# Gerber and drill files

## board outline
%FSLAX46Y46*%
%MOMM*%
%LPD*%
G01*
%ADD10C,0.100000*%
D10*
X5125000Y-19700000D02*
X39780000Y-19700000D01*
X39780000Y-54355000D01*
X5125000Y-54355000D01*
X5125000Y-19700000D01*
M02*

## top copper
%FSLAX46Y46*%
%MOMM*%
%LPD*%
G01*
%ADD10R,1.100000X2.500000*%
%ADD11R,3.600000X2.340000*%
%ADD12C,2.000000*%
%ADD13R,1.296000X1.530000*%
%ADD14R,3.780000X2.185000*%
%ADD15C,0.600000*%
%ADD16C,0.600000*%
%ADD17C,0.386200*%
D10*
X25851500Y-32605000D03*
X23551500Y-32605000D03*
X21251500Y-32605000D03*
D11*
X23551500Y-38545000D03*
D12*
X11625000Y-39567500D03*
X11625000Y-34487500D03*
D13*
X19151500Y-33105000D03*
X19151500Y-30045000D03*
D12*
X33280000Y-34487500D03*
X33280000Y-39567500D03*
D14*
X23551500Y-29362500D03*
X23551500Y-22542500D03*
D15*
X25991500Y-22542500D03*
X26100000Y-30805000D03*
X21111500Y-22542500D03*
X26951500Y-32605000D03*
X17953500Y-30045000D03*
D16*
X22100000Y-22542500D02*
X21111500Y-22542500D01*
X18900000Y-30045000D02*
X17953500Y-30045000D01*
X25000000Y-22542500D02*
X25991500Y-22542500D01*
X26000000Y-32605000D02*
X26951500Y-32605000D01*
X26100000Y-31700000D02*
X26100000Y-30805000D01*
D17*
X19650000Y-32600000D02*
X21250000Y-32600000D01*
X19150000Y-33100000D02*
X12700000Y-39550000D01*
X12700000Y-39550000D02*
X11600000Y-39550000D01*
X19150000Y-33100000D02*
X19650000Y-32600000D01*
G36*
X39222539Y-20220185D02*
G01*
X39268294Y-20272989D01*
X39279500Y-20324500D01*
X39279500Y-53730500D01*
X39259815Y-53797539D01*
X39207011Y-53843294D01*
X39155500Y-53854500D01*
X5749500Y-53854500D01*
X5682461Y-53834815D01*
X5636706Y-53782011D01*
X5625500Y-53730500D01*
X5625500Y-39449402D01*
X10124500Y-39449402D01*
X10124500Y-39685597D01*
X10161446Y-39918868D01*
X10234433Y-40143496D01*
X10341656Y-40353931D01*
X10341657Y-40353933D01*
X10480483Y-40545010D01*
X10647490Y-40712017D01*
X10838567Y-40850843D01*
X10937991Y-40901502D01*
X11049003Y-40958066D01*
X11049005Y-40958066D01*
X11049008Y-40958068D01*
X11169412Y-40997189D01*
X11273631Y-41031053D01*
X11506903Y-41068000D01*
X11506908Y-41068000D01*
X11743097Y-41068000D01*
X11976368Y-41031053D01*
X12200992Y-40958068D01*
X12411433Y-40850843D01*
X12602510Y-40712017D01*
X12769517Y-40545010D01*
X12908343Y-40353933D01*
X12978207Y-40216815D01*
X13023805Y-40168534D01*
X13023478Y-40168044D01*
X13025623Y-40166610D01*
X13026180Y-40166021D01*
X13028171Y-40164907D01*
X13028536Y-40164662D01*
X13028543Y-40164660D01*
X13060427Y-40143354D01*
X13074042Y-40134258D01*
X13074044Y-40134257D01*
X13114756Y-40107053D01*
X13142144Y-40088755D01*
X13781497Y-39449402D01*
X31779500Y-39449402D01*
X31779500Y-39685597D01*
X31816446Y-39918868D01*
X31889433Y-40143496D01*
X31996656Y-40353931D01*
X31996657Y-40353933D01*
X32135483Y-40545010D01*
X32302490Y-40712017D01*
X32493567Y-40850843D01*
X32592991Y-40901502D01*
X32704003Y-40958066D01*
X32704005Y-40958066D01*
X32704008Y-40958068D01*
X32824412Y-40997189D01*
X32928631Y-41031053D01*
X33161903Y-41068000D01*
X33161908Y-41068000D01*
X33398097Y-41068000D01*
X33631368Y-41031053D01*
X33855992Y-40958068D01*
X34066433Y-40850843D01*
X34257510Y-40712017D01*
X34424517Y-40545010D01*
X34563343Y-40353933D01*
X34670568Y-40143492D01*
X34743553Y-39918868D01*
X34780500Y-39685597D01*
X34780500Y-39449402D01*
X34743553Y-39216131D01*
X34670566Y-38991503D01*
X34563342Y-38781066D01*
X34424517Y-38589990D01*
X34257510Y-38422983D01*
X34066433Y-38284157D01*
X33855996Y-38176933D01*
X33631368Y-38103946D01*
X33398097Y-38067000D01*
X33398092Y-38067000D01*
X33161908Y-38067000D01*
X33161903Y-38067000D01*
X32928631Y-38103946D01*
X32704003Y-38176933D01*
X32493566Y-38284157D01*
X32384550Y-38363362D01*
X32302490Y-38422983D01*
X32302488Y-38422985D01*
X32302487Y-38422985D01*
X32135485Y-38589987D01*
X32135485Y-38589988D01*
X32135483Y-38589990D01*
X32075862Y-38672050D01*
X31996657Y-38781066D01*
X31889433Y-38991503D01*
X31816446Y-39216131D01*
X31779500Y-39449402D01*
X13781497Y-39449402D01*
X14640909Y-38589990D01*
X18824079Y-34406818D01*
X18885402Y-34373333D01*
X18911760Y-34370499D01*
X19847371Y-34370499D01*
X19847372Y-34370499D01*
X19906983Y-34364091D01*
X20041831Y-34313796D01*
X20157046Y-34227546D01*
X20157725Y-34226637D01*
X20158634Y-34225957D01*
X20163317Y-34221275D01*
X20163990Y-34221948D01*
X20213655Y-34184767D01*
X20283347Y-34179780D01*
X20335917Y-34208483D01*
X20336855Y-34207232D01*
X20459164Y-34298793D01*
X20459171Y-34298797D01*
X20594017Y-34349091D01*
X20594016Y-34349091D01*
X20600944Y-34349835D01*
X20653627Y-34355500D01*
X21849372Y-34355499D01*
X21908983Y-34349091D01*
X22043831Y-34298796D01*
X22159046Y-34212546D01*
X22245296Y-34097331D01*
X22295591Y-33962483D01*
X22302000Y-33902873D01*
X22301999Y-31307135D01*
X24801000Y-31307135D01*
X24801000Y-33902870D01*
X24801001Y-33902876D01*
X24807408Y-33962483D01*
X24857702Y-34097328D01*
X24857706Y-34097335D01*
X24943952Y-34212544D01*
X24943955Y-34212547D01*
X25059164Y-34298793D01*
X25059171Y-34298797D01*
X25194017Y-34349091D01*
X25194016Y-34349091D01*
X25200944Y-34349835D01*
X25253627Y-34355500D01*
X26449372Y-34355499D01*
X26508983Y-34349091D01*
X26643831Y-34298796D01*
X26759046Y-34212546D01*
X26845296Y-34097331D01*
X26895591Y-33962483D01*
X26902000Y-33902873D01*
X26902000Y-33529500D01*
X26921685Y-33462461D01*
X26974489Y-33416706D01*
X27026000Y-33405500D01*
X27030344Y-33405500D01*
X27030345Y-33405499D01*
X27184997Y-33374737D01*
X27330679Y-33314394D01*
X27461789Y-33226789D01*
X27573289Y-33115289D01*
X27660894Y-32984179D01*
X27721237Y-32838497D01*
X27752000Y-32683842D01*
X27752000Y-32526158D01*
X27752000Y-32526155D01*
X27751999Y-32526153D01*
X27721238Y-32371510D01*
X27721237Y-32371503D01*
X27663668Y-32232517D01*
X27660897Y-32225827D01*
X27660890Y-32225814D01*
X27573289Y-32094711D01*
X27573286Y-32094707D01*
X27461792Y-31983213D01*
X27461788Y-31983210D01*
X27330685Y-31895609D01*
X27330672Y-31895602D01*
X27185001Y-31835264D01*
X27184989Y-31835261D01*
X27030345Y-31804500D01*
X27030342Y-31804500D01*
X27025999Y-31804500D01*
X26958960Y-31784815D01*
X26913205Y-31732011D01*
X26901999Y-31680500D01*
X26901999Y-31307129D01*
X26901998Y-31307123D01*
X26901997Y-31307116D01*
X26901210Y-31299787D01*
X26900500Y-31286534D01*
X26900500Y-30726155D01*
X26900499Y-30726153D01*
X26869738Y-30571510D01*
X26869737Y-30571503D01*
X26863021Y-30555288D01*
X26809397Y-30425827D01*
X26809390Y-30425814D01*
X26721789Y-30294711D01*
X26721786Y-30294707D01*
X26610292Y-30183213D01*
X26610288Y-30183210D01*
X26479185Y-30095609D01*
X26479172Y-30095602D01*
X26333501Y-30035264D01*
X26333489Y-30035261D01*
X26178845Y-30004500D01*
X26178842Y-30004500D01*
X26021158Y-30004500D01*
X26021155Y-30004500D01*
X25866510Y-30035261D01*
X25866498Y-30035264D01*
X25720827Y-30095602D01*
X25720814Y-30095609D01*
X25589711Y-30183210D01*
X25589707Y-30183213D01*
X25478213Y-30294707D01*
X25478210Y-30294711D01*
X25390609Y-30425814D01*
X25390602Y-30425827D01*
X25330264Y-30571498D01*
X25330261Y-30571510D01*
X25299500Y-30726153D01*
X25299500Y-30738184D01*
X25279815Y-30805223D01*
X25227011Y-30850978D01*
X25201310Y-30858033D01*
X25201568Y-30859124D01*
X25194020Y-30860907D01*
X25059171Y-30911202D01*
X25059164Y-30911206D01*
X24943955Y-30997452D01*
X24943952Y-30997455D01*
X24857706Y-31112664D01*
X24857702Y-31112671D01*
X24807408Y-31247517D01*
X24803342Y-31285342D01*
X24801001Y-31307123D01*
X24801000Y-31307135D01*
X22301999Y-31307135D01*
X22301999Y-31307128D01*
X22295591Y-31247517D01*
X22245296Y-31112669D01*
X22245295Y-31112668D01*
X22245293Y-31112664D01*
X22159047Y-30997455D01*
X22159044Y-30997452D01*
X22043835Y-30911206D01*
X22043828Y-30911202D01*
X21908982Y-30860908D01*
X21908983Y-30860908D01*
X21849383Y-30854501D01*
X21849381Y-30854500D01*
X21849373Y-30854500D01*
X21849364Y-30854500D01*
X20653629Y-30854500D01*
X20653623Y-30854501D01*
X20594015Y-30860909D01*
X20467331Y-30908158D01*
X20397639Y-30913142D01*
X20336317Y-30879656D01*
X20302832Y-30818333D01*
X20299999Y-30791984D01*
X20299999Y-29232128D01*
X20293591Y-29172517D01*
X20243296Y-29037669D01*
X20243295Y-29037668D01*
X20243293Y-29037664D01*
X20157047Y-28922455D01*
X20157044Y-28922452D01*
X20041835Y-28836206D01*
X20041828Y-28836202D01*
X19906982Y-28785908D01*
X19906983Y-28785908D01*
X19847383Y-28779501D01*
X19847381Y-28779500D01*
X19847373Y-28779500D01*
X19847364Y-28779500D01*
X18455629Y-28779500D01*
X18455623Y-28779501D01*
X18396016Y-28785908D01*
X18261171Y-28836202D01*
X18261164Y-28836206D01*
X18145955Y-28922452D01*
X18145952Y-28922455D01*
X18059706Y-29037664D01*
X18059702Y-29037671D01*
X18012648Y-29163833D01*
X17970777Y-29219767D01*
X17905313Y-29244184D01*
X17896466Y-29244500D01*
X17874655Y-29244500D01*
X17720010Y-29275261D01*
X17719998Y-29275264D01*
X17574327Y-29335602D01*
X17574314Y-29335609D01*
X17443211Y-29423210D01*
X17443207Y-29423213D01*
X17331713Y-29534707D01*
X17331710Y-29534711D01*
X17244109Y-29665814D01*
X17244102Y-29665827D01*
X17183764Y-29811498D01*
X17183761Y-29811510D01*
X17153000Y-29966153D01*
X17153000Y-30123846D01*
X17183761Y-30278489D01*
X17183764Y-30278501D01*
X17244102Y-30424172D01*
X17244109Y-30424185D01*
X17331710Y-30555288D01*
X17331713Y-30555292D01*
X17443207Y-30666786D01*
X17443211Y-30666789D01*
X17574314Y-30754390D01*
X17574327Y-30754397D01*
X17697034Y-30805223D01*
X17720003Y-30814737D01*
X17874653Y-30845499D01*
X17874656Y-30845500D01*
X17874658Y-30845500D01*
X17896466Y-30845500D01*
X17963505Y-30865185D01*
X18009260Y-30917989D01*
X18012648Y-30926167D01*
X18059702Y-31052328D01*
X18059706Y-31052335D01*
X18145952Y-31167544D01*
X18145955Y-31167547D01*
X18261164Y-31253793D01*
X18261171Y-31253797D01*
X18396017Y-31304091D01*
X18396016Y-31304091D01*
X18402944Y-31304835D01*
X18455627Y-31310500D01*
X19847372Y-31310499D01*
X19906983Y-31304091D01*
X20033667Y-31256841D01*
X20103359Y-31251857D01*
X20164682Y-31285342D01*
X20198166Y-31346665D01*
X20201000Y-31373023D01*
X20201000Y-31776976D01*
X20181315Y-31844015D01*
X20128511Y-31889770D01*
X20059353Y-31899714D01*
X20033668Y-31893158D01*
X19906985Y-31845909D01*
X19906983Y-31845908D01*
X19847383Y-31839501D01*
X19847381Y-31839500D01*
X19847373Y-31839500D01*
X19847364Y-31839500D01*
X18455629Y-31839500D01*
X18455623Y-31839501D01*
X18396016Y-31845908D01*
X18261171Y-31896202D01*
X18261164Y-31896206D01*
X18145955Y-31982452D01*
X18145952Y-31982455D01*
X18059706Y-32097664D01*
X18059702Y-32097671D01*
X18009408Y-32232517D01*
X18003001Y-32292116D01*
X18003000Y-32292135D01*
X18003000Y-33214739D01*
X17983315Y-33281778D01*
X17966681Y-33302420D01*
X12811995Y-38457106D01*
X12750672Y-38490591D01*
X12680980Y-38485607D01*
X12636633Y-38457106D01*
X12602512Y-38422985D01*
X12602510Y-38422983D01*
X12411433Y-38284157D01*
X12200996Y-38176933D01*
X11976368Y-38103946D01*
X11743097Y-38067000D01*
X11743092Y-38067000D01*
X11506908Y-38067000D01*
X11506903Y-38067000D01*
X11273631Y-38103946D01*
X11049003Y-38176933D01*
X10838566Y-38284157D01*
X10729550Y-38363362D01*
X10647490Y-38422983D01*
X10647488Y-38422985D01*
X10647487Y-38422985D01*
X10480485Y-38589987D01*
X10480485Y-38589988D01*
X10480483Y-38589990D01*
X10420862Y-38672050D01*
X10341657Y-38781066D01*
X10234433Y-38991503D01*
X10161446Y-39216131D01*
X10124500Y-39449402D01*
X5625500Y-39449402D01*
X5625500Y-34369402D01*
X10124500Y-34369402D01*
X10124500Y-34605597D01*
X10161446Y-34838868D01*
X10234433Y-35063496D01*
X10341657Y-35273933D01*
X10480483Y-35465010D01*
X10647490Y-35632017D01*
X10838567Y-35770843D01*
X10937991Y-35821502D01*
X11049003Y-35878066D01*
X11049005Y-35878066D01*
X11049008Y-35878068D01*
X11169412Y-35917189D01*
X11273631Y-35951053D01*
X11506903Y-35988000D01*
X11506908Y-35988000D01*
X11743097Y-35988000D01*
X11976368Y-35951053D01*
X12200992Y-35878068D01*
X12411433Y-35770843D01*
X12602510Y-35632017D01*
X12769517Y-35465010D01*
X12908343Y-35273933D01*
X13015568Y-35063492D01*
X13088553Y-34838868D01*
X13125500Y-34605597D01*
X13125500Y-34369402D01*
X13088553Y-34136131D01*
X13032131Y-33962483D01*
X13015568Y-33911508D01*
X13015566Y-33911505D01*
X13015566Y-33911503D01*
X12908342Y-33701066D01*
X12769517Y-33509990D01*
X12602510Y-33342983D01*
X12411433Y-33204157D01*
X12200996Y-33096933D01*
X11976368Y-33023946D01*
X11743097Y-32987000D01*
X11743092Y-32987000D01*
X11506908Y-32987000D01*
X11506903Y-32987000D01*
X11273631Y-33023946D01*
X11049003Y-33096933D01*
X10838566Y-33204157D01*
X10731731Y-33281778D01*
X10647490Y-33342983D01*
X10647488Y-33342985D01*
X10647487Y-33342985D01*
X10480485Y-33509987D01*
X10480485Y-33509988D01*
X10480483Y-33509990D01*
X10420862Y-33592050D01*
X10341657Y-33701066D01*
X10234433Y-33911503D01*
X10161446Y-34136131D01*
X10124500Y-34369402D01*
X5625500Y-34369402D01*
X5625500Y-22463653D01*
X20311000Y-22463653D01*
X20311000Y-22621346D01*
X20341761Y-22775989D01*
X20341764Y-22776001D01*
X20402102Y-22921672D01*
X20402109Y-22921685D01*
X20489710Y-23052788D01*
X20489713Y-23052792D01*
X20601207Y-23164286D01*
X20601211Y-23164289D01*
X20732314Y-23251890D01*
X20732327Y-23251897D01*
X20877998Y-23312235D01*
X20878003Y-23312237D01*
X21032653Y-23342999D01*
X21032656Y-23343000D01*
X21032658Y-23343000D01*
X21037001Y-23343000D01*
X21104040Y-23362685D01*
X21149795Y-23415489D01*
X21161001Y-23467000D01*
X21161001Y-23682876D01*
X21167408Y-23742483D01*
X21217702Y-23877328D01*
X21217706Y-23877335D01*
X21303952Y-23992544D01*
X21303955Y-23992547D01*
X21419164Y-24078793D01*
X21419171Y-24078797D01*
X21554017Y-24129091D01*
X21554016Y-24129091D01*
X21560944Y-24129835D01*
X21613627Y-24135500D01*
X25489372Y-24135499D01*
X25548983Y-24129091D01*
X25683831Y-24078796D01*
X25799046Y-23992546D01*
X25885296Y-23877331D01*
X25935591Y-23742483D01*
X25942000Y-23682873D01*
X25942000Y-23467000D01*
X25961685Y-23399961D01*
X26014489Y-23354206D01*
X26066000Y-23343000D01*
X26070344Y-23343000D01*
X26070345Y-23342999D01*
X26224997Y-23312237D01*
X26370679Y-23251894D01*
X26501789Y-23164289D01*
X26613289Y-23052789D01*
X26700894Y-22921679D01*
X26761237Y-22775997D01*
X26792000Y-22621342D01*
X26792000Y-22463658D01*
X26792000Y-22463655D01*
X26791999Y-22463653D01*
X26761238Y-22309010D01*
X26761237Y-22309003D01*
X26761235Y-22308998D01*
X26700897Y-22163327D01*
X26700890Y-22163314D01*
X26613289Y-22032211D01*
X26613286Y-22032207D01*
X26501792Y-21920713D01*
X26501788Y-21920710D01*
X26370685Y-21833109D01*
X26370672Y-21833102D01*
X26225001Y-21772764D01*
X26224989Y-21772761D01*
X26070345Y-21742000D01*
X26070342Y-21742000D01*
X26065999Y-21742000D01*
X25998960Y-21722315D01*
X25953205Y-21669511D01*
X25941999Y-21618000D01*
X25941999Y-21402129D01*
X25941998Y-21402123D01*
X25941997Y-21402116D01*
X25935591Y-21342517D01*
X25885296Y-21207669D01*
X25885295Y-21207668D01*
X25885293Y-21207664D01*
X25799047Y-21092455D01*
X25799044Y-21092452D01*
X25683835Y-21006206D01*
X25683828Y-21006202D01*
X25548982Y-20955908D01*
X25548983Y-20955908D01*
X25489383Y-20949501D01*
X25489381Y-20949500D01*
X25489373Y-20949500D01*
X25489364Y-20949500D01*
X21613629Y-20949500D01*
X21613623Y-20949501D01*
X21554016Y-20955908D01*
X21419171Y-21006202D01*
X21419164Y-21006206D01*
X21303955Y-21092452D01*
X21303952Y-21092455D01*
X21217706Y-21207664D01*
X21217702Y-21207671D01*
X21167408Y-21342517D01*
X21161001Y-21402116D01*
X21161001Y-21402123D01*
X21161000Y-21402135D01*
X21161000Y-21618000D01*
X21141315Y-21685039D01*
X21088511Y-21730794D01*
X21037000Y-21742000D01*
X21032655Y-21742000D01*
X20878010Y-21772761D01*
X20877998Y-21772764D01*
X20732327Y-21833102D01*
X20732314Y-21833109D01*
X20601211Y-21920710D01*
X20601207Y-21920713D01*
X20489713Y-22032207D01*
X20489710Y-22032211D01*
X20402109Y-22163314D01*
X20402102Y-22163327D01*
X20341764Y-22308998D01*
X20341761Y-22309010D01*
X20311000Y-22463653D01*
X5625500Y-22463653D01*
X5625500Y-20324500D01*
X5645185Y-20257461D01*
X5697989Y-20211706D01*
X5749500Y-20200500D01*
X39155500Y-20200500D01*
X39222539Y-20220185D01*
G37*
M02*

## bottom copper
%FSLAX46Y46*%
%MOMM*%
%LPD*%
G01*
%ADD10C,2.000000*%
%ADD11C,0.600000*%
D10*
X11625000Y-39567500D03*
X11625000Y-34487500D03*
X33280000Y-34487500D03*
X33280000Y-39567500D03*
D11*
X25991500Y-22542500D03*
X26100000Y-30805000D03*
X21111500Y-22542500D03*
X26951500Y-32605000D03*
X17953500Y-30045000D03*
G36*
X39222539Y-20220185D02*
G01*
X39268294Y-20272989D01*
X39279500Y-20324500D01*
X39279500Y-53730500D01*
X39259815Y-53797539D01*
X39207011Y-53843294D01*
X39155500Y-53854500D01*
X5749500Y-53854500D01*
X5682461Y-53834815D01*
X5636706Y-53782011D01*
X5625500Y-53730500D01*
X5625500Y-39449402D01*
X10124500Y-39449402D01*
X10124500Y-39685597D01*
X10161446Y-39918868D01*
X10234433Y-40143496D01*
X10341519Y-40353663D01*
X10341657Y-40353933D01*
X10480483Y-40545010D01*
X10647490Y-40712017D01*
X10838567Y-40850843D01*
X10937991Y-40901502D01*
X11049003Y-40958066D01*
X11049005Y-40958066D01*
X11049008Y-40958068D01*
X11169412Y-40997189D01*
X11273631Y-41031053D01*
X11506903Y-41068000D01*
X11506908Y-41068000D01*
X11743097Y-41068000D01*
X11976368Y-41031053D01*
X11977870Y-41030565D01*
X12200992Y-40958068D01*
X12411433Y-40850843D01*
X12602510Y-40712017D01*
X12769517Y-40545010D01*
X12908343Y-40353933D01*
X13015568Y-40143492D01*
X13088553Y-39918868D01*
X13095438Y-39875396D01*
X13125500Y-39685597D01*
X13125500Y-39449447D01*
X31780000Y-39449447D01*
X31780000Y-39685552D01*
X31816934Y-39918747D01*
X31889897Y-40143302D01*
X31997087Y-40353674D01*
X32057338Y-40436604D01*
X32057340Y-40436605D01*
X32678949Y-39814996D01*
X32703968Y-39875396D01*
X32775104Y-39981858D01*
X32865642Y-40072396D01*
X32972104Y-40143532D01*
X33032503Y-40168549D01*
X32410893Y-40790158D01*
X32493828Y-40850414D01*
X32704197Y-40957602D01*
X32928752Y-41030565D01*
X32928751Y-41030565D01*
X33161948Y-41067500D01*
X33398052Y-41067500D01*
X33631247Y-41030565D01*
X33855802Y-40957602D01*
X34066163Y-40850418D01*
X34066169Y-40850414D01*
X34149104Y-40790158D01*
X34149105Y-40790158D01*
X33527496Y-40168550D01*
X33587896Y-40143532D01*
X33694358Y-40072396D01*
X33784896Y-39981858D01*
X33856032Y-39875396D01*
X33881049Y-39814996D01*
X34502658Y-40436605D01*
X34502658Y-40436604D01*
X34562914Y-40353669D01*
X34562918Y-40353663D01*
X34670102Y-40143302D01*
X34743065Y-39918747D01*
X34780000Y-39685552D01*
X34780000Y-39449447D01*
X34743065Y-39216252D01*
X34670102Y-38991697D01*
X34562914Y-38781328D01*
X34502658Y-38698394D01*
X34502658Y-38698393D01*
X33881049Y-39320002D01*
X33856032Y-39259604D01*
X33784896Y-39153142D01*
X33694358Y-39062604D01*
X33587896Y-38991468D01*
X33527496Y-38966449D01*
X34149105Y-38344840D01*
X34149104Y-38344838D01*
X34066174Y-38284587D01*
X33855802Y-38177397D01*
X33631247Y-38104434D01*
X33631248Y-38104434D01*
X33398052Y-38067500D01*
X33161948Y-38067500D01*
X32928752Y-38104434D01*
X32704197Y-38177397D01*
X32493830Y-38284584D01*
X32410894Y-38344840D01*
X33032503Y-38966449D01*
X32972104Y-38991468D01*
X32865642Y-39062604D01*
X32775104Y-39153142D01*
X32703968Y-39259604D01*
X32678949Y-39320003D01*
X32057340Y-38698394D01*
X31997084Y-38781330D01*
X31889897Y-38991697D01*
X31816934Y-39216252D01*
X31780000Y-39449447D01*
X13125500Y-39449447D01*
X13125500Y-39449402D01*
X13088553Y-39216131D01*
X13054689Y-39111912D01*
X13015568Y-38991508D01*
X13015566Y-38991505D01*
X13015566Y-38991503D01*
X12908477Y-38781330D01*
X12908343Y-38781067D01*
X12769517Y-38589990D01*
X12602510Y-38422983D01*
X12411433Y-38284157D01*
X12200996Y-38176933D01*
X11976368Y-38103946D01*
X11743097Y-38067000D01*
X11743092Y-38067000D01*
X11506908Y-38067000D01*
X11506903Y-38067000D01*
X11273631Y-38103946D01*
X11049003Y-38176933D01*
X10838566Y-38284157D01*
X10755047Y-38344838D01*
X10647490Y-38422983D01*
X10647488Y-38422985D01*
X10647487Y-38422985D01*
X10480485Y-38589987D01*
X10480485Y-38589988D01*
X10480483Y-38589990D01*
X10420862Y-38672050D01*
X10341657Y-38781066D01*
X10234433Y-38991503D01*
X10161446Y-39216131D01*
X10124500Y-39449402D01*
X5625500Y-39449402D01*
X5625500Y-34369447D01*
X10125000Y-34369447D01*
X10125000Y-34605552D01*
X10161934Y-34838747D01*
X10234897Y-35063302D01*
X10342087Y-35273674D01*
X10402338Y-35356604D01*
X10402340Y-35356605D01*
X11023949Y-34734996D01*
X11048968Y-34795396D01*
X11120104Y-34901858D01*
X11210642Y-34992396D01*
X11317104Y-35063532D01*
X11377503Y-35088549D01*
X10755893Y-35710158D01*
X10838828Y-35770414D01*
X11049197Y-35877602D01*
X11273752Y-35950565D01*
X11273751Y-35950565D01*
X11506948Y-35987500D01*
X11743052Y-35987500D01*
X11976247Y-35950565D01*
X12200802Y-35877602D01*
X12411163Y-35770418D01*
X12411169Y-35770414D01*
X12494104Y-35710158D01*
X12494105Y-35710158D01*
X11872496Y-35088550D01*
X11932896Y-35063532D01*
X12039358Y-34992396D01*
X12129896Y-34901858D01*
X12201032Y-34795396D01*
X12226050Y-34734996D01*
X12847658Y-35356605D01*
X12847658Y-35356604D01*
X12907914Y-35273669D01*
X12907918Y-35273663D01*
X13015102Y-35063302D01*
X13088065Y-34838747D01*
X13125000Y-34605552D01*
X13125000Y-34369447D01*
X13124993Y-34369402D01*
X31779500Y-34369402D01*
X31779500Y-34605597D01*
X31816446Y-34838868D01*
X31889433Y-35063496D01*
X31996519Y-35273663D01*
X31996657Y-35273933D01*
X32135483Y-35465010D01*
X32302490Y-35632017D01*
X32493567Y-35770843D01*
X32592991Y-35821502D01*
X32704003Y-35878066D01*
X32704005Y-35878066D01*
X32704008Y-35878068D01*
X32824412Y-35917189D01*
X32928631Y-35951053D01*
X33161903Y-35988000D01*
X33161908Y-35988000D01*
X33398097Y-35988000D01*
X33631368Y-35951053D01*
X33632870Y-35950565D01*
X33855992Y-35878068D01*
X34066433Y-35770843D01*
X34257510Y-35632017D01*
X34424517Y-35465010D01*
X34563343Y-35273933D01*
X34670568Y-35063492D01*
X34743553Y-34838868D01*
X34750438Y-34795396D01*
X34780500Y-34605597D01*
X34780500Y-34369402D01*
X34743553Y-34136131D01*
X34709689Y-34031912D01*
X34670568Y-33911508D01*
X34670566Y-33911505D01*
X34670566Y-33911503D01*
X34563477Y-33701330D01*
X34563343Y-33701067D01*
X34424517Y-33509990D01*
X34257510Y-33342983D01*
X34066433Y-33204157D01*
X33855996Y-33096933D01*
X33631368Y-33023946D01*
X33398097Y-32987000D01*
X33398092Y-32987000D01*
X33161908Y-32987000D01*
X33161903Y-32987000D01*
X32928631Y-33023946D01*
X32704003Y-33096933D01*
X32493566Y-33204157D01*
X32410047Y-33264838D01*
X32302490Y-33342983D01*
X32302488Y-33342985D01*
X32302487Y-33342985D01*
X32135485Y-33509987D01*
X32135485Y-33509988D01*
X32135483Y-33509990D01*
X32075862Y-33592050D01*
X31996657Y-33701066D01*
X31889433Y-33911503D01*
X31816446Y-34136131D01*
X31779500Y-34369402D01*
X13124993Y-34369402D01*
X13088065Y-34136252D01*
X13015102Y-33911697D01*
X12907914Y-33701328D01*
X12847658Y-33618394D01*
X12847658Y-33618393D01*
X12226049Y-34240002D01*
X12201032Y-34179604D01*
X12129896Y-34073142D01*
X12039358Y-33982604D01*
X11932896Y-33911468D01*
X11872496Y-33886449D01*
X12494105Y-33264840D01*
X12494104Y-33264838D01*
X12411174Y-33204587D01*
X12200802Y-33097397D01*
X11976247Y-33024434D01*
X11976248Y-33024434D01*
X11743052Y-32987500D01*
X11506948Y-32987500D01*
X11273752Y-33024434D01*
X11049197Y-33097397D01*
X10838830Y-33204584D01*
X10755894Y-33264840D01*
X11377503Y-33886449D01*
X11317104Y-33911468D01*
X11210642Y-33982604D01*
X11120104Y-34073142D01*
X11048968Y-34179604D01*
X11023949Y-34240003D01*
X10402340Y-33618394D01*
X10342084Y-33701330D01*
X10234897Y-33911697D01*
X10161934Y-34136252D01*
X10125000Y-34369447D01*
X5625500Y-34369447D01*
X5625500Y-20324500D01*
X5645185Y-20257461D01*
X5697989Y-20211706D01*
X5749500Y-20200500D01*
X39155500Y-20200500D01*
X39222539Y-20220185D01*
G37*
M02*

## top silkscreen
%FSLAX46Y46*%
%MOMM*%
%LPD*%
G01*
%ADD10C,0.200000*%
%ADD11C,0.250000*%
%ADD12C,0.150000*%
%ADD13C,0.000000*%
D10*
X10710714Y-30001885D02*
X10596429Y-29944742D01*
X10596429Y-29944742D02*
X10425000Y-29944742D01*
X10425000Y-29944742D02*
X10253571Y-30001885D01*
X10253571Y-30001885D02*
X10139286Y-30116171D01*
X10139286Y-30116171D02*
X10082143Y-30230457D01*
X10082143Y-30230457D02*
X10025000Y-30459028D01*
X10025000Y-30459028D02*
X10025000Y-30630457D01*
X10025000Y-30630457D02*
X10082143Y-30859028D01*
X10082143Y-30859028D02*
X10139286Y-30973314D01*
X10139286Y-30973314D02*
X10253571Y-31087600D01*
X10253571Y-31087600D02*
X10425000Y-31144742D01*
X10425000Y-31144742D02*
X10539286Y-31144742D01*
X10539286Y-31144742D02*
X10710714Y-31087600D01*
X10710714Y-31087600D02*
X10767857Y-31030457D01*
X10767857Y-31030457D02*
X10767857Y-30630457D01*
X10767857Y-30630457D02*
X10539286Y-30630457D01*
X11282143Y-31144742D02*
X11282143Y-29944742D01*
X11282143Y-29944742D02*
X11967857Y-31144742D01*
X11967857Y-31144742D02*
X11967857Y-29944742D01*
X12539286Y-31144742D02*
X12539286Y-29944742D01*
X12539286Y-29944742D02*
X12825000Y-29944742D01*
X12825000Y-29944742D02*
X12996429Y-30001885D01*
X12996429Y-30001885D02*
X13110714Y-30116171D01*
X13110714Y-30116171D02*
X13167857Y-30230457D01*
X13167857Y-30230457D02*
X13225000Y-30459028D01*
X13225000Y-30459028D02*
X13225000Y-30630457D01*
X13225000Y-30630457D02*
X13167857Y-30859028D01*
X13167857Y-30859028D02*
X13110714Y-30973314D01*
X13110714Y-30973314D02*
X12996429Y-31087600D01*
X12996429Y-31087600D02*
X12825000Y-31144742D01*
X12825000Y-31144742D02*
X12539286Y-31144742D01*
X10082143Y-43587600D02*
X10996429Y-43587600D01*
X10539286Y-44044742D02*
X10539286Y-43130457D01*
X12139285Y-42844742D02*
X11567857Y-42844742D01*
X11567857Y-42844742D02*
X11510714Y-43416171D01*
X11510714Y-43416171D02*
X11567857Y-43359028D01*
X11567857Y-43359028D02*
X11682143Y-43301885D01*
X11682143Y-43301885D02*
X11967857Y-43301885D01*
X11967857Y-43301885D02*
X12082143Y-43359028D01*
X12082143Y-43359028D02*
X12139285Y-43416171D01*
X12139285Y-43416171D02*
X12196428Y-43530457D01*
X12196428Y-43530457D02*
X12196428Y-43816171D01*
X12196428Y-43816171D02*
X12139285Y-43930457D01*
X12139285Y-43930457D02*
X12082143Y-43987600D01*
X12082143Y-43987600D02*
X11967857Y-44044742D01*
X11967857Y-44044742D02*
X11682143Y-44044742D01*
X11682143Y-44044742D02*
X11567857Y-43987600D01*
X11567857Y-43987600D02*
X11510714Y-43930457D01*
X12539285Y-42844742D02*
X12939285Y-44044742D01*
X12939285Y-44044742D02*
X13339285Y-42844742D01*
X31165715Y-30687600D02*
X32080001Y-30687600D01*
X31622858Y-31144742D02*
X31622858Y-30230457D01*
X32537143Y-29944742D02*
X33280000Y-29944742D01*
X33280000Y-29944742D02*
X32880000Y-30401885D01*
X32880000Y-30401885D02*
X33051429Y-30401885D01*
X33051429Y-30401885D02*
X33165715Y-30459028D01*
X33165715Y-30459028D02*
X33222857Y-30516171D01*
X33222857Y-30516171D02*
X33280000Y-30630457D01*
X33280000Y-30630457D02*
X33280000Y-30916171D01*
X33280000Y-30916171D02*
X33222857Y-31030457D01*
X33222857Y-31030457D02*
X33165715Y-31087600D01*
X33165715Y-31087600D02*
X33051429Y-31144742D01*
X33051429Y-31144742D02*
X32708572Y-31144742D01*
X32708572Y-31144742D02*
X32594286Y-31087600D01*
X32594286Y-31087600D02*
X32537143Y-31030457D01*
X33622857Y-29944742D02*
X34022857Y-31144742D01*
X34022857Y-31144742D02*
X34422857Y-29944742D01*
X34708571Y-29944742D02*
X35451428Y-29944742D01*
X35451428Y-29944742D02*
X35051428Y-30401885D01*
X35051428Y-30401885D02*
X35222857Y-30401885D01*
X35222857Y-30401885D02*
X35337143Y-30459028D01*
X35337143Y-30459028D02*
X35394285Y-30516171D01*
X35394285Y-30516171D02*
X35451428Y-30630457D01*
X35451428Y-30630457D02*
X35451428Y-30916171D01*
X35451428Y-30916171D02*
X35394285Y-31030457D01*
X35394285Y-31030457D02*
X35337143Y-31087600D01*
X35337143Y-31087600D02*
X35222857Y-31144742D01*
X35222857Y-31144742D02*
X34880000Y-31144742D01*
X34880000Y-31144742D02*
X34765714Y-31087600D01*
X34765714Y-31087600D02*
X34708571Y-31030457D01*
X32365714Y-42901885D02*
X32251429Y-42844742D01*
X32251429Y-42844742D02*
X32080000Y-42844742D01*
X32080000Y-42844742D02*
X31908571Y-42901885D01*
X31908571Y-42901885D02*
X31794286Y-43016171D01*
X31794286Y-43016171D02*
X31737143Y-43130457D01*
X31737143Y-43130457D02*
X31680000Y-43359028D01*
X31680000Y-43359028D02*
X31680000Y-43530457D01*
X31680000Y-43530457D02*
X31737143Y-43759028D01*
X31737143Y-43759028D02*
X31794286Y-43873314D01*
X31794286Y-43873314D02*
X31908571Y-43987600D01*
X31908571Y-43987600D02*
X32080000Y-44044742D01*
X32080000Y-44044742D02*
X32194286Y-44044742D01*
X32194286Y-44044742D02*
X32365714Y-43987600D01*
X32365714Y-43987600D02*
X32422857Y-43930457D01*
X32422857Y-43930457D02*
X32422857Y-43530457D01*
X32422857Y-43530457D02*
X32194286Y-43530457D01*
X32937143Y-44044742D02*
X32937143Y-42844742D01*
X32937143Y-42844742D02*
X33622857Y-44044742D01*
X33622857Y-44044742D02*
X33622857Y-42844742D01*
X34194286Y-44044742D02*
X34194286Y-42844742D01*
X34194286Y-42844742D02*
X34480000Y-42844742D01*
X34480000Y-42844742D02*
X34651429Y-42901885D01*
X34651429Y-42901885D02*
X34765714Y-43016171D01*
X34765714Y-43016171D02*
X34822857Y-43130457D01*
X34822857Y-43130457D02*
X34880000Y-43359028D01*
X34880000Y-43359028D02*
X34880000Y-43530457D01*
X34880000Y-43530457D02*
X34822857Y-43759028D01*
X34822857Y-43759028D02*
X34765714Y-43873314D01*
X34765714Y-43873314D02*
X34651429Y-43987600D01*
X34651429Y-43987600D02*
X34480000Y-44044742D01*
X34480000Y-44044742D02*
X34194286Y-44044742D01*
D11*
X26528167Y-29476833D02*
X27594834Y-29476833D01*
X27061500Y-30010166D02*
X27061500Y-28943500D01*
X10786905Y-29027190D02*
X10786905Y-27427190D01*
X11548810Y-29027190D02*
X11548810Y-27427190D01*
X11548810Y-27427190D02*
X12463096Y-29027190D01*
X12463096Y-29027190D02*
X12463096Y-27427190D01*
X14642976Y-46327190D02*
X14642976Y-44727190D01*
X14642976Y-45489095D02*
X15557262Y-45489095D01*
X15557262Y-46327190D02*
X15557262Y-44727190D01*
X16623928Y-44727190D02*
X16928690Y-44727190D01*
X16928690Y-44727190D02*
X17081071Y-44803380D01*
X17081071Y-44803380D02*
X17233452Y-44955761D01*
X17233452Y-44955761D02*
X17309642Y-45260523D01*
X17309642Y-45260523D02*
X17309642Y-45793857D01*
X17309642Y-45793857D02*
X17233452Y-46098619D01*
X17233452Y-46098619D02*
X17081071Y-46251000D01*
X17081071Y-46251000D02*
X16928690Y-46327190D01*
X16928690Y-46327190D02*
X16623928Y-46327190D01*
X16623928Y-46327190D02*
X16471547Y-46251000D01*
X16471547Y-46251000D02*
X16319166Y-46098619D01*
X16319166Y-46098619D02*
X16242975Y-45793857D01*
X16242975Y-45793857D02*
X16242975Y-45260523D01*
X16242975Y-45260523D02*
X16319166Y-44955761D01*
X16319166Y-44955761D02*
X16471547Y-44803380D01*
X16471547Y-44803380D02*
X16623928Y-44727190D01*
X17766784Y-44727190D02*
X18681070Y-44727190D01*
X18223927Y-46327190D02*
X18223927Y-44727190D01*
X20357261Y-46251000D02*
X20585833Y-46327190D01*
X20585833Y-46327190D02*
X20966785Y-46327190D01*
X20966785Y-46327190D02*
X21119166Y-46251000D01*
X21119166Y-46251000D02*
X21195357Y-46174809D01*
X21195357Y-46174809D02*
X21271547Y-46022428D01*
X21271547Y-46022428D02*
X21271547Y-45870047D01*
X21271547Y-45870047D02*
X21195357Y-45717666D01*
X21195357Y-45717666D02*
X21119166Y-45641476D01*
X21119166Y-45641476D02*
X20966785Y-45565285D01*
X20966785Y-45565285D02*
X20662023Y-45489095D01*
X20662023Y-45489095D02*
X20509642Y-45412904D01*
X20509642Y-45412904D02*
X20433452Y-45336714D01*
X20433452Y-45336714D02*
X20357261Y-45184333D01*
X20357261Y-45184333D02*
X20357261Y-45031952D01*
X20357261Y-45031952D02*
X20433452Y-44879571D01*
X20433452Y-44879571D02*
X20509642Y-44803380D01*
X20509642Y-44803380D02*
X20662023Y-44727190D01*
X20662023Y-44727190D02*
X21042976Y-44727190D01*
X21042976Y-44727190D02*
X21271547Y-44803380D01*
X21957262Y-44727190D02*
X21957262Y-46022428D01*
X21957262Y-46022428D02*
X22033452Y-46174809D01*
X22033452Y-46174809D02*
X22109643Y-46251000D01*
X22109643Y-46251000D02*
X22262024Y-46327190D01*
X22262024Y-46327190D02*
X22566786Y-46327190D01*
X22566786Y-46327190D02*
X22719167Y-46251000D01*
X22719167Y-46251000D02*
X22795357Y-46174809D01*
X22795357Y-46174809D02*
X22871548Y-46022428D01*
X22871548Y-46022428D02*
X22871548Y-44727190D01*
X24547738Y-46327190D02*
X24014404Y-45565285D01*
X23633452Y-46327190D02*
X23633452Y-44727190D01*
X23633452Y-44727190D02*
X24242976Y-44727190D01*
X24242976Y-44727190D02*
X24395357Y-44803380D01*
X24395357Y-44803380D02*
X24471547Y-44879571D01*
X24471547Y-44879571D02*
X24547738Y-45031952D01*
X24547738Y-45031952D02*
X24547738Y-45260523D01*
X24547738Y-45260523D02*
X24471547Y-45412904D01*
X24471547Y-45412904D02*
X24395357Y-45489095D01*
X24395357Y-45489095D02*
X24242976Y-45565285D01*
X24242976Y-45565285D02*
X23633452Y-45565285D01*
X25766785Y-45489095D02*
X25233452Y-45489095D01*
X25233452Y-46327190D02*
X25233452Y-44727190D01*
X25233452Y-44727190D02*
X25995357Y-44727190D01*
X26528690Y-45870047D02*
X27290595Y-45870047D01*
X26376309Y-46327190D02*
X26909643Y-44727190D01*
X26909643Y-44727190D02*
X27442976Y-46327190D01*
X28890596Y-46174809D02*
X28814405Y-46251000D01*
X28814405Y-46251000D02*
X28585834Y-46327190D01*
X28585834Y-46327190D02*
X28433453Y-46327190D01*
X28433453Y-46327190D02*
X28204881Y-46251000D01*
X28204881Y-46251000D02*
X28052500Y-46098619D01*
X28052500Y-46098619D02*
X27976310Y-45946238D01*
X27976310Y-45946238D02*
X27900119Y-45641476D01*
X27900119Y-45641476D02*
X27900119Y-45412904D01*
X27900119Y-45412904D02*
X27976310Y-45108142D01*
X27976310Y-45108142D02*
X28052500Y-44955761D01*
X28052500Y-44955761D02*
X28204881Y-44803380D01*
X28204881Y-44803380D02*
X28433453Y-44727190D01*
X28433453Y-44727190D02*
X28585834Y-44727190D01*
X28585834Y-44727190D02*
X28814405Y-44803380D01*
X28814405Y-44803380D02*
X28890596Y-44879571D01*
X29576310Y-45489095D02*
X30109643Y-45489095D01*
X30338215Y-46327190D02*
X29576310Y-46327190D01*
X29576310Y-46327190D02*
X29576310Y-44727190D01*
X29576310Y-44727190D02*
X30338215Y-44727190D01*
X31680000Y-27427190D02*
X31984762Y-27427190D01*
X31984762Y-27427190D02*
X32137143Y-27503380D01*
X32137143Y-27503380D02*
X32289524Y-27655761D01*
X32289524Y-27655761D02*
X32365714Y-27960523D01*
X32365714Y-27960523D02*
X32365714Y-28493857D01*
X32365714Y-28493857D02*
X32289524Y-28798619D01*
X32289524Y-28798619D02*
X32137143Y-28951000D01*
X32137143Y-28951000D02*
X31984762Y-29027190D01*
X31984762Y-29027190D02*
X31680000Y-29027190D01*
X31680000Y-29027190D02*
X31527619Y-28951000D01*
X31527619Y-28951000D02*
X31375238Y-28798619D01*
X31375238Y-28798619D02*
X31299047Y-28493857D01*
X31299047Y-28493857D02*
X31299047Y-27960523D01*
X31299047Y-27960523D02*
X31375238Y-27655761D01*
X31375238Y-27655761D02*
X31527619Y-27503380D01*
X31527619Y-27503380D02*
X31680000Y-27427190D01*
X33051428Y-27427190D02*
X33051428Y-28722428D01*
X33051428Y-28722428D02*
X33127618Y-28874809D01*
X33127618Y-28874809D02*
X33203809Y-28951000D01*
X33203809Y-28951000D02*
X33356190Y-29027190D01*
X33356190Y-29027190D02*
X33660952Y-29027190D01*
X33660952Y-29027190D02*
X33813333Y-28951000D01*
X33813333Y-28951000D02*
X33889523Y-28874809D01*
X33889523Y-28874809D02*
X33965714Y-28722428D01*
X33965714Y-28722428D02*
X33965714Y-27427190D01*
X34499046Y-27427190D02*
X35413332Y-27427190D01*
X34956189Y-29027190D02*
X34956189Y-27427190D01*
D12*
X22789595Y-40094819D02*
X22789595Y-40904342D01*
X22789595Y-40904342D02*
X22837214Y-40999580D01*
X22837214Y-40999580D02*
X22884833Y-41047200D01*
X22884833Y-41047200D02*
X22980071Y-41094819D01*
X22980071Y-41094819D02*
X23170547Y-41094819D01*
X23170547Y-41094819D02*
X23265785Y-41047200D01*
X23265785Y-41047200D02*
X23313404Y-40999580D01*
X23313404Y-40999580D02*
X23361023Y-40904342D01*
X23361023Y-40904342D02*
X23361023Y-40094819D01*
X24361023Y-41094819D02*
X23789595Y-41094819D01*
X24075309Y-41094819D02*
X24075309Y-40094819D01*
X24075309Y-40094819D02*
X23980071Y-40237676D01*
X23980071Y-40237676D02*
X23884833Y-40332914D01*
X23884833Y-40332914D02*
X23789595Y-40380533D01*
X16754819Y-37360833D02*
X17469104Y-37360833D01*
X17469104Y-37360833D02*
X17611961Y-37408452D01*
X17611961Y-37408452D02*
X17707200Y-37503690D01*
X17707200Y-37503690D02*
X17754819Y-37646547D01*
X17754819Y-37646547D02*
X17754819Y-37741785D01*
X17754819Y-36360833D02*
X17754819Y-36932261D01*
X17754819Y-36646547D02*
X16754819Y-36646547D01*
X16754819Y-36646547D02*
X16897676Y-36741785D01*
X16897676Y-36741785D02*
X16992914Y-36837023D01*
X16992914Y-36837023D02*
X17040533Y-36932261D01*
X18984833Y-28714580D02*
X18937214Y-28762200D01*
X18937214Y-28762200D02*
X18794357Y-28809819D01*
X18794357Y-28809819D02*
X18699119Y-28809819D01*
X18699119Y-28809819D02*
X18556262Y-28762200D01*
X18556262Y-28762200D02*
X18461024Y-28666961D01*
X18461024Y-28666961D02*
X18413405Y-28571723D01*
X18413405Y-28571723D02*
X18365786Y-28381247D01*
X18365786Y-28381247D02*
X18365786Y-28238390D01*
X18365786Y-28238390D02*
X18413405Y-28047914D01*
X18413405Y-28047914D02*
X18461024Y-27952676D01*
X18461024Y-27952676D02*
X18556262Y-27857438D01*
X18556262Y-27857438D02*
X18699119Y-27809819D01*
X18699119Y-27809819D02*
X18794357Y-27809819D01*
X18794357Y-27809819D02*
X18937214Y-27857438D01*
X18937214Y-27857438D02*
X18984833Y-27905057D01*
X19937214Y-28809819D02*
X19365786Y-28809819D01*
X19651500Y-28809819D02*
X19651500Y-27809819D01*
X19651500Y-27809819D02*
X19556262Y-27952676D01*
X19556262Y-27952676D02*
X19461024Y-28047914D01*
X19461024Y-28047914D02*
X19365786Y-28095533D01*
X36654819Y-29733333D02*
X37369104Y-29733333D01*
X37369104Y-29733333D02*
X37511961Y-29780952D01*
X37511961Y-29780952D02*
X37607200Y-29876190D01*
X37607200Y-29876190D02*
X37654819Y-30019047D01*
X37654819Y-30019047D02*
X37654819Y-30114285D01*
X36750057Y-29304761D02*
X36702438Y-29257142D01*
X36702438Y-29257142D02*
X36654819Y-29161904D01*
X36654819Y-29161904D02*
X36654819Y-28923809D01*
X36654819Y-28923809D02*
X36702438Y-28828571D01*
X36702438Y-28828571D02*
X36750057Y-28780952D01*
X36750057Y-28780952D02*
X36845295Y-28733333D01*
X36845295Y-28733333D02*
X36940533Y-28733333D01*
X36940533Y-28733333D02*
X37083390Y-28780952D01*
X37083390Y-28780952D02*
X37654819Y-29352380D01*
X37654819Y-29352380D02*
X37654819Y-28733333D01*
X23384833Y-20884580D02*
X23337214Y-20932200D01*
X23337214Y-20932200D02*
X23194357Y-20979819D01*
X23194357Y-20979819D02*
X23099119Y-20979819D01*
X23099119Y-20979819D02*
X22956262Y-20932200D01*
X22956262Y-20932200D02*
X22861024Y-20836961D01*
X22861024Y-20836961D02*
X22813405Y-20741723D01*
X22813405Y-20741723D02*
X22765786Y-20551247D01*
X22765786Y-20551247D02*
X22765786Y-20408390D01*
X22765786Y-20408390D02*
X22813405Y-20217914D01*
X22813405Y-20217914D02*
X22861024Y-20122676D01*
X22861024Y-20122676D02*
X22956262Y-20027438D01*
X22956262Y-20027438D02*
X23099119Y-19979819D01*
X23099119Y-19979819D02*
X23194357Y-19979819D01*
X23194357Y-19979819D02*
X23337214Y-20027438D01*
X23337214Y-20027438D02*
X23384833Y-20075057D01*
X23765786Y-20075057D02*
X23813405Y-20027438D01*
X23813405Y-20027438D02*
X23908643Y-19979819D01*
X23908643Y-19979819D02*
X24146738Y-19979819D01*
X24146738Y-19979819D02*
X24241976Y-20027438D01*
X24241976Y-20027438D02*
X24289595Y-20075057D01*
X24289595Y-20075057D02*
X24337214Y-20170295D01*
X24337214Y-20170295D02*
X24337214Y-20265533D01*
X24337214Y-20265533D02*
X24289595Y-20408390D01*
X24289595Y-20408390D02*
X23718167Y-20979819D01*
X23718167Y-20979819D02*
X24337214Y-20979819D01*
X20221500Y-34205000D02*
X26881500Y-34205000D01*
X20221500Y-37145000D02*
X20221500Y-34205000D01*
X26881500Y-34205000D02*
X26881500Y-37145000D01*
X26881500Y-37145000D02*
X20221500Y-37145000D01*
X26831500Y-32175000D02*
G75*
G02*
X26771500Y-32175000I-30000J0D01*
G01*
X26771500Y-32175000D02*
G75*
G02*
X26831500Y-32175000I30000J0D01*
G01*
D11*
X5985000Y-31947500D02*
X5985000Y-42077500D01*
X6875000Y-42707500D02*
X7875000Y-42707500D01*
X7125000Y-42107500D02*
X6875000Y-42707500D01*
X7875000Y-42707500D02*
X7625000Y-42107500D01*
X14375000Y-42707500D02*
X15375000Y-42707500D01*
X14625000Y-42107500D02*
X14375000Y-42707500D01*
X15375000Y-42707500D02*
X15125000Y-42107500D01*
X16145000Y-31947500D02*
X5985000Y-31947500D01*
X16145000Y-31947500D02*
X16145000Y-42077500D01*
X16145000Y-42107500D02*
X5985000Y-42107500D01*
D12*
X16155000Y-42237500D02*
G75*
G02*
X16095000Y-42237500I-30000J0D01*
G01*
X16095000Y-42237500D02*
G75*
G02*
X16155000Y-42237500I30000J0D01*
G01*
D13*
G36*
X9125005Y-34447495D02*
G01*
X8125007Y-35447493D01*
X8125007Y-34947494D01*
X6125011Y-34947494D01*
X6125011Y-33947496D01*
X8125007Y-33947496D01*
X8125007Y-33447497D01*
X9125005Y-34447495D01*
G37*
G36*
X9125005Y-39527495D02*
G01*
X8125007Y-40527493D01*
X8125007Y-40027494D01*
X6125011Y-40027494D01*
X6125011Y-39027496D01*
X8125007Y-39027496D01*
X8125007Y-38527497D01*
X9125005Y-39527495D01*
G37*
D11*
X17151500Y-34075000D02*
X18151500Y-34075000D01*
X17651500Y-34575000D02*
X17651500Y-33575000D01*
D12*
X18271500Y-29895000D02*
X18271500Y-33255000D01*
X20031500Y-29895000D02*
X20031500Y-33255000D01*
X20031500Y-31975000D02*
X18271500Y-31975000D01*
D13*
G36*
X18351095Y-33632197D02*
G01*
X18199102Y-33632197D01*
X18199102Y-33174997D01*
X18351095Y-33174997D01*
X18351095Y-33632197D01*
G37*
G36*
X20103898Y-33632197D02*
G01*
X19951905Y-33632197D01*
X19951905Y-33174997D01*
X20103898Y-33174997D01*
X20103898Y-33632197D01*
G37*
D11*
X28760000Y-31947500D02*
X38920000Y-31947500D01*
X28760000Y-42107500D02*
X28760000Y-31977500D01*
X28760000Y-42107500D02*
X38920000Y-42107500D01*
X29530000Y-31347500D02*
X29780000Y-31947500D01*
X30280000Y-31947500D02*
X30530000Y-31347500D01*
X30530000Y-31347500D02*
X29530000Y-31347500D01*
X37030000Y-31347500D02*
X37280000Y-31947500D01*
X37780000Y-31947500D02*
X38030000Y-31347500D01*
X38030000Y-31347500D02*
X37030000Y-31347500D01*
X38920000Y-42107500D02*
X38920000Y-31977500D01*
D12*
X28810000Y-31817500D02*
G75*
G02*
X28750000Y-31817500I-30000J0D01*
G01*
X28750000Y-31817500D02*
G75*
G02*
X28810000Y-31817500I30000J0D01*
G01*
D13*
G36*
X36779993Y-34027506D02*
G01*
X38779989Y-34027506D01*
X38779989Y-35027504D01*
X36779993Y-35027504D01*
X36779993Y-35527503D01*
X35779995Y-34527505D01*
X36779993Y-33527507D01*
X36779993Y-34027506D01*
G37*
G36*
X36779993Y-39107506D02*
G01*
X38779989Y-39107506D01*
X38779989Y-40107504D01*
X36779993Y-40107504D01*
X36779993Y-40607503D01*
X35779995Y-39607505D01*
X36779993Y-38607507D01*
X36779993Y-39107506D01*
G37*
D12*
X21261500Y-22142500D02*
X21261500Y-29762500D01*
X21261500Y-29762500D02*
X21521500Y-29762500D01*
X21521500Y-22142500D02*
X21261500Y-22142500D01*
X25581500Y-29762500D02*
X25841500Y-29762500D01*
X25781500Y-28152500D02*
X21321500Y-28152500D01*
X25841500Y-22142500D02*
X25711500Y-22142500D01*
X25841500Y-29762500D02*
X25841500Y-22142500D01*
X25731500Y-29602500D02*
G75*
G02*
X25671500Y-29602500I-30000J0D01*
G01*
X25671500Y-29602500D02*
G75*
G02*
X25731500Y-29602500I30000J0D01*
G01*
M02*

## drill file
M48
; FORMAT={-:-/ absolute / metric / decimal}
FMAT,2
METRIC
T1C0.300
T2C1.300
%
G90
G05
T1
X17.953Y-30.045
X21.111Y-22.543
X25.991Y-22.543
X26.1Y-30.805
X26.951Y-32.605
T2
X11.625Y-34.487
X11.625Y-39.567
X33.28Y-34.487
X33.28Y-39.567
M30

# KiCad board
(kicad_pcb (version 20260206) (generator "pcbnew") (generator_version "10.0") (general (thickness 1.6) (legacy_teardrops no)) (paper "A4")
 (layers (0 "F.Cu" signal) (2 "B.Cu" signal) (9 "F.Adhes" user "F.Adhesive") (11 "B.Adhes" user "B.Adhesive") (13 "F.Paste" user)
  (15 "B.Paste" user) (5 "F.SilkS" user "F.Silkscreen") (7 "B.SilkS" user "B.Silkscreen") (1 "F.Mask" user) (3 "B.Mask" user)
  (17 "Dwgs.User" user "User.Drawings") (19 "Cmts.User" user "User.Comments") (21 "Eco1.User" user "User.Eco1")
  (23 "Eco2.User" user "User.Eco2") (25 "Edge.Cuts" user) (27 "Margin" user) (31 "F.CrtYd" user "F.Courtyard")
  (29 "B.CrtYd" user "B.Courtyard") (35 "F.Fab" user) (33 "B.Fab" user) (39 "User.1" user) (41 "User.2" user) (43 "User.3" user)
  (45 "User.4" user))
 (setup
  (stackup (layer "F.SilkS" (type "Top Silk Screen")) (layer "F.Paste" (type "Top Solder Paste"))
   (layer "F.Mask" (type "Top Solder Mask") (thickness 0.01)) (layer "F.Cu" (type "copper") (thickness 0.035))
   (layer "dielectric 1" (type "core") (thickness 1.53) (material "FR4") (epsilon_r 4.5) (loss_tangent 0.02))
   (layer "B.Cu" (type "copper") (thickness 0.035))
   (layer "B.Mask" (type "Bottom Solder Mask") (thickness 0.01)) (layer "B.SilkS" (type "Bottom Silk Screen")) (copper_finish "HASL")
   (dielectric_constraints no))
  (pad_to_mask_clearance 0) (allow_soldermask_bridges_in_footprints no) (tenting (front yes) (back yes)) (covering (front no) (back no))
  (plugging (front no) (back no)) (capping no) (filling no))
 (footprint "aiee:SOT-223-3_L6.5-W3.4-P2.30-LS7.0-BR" (layer "F.Cu") (at 23.5515 35.575 90)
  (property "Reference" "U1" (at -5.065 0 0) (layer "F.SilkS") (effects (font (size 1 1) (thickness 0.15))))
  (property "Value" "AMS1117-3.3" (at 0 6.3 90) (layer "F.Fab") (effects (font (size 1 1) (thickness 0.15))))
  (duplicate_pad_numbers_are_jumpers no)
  (fp_line (start 1.37 -3.33) (end 1.37 3.33) (stroke (width 0.15) (type solid)) (layer "F.SilkS"))
  (fp_line (start -1.57 -3.33) (end 1.37 -3.33) (stroke (width 0.15) (type solid)) (layer "F.SilkS"))
  (fp_line (start 1.37 3.33) (end -1.57 3.33) (stroke (width 0.15) (type solid)) (layer "F.SilkS"))
  (fp_line (start -1.57 3.33) (end -1.57 -3.33) (stroke (width 0.15) (type solid)) (layer "F.SilkS"))
  (fp_circle (center 3.4 3.25) (end 3.43 3.25) (stroke (width 0.15) (type solid)) (fill no) (layer "F.SilkS"))
  (pad "1" smd rect (at 2.97 2.3 90) (size 2.5 1.1) (layers "F.Cu" "F.Mask" "F.Paste") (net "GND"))
  (pad "2" smd rect (at 2.97 0 90) (size 2.5 1.1) (layers "F.Cu" "F.Mask" "F.Paste") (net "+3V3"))
  (pad "3" smd rect (at 2.97 -2.3 90) (size 2.5 1.1) (layers "F.Cu" "F.Mask" "F.Paste") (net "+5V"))
  (pad "4" smd rect (at -2.97 0 90) (size 2.34 3.6) (layers "F.Cu" "F.Mask" "F.Paste") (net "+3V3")))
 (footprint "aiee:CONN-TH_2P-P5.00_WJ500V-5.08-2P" (layer "F.Cu") (at 11.625 37.0275 90)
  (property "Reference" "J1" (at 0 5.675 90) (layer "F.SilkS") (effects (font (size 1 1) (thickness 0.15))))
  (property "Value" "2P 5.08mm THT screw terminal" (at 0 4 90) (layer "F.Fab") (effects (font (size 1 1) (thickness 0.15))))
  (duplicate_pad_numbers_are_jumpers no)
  (fp_line (start 5.08 -5.64) (end -5.05 -5.64) (stroke (width 0.25) (type solid)) (layer "F.SilkS"))
  (fp_line (start -5.68 -4.75) (end -5.68 -3.75) (stroke (width 0.25) (type solid)) (layer "F.SilkS"))
  (fp_line (start -5.08 -4.5) (end -5.68 -4.75) (stroke (width 0.25) (type solid)) (layer "F.SilkS"))
  (fp_line (start -5.68 -3.75) (end -5.08 -4) (stroke (width 0.25) (type solid)) (layer "F.SilkS"))
  (fp_line (start -5.68 2.75) (end -5.68 3.75) (stroke (width 0.25) (type solid)) (layer "F.SilkS"))
  (fp_line (start -5.08 3) (end -5.68 2.75) (stroke (width 0.25) (type solid)) (layer "F.SilkS"))
  (fp_line (start -5.68 3.75) (end -5.08 3.5) (stroke (width 0.25) (type solid)) (layer "F.SilkS"))
  (fp_line (start 5.08 4.52) (end 5.08 -5.64) (stroke (width 0.25) (type solid)) (layer "F.SilkS"))
  (fp_line (start 5.08 4.52) (end -5.05 4.52) (stroke (width 0.25) (type solid)) (layer "F.SilkS"))
  (fp_line (start -5.08 4.52) (end -5.08 -5.64) (stroke (width 0.25) (type solid)) (layer "F.SilkS"))
  (fp_circle (center -5.21 4.5) (end -5.18 4.5) (stroke (width 0.15) (type solid)) (fill no) (layer "F.SilkS"))
  (fp_poly
   (pts (xy 2.080006 -5.499989) (xy 3.080004 -5.499989) (xy 3.080004 -3.499993) (xy 3.580003 -3.499993) (xy 2.580005 -2.499995)
    (xy 1.580007 -3.499993) (xy 2.080006 -3.499993) (xy 2.080006 -5.499989))
   (stroke (width 0) (type solid)) (fill yes) (layer "F.SilkS"))
  (fp_poly
   (pts (xy -2.999994 -5.499989) (xy -1.999996 -5.499989) (xy -1.999996 -3.499993) (xy -1.499997 -3.499993) (xy -2.499995 -2.499995)
    (xy -3.499993 -3.499993) (xy -2.999994 -3.499993) (xy -2.999994 -5.499989))
   (stroke (width 0) (type solid)) (fill yes) (layer "F.SilkS"))
  (pad "1" thru_hole circle (at -2.54 0 270) (size 2 2) (drill 1.300022) (layers "*.Cu" "*.Mask") (remove_unused_layers no) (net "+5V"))
  (pad "2" thru_hole circle (at 2.54 0 270) (size 2 2) (drill 1.300022) (layers "*.Cu" "*.Mask") (remove_unused_layers no) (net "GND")))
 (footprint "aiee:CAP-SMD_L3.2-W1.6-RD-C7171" (layer "F.Cu") (at 19.1515 31.575 90)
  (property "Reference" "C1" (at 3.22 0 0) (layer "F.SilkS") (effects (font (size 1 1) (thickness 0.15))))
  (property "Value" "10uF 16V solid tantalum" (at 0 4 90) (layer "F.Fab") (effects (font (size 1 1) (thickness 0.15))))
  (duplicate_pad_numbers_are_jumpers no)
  (fp_line (start -2.5 -2) (end -2.5 -1) (stroke (width 0.25) (type solid)) (layer "F.SilkS"))
  (fp_line (start -3 -1.5) (end -2 -1.5) (stroke (width 0.25) (type solid)) (layer "F.SilkS"))
  (fp_line (start 1.68 -0.88) (end -1.68 -0.88) (stroke (width 0.15) (type solid)) (layer "F.SilkS"))
  (fp_line (start 1.68 0.88) (end -1.68 0.88) (stroke (width 0.15) (type solid)) (layer "F.SilkS"))
  (fp_line (start -0.4 0.88) (end -0.4 -0.88) (stroke (width 0.15) (type solid)) (layer "F.SilkS"))
  (fp_poly
   (pts (xy -1.599997 -0.952398) (xy -1.599997 -0.800405) (xy -2.057197 -0.800405) (xy -2.057197 -0.952398) (xy -1.599997 -0.952398))
   (stroke (width 0) (type solid)) (fill yes) (layer "F.SilkS"))
  (fp_poly
   (pts (xy -1.599997 0.952398) (xy -1.599997 0.800405) (xy -2.057197 0.800405) (xy -2.057197 0.952398) (xy -1.599997 0.952398))
   (stroke (width 0) (type solid)) (fill yes) (layer "F.SilkS"))
  (pad "1" smd rect (at -1.53 0 270) (size 1.53 1.296) (layers "F.Cu" "F.Mask" "F.Paste") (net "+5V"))
  (pad "2" smd rect (at 1.53 0 270) (size 1.53 1.296) (layers "F.Cu" "F.Mask" "F.Paste") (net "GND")))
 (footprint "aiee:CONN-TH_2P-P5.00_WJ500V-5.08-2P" (layer "F.Cu") (at 33.28 37.0275 -90)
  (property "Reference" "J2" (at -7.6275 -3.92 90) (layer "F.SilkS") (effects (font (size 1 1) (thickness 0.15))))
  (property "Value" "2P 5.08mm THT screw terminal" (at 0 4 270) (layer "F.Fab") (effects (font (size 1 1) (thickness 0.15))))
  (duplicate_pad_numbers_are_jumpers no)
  (fp_line (start -5.08 4.52) (end -5.08 -5.64) (stroke (width 0.25) (type solid)) (layer "F.SilkS"))
  (fp_line (start 5.08 4.52) (end -5.05 4.52) (stroke (width 0.25) (type solid)) (layer "F.SilkS"))
  (fp_line (start 5.08 4.52) (end 5.08 -5.64) (stroke (width 0.25) (type solid)) (layer "F.SilkS"))
  (fp_line (start -5.68 3.75) (end -5.08 3.5) (stroke (width 0.25) (type solid)) (layer "F.SilkS"))
  (fp_line (start -5.08 3) (end -5.68 2.75) (stroke (width 0.25) (type solid)) (layer "F.SilkS"))
  (fp_line (start -5.68 2.75) (end -5.68 3.75) (stroke (width 0.25) (type solid)) (layer "F.SilkS"))
  (fp_line (start -5.68 -3.75) (end -5.08 -4) (stroke (width 0.25) (type solid)) (layer "F.SilkS"))
  (fp_line (start -5.08 -4.5) (end -5.68 -4.75) (stroke (width 0.25) (type solid)) (layer "F.SilkS"))
  (fp_line (start -5.68 -4.75) (end -5.68 -3.75) (stroke (width 0.25) (type solid)) (layer "F.SilkS"))
  (fp_line (start 5.08 -5.64) (end -5.05 -5.64) (stroke (width 0.25) (type solid)) (layer "F.SilkS"))
  (fp_circle (center -5.21 4.5) (end -5.18 4.5) (stroke (width 0.15) (type solid)) (fill no) (layer "F.SilkS"))
  (fp_poly
   (pts (xy -2.999994 -5.499989) (xy -1.999996 -5.499989) (xy -1.999996 -3.499993) (xy -1.499997 -3.499993) (xy -2.499995 -2.499995)
    (xy -3.499993 -3.499993) (xy -2.999994 -3.499993) (xy -2.999994 -5.499989))
   (stroke (width 0) (type solid)) (fill yes) (layer "F.SilkS"))
  (fp_poly
   (pts (xy 2.080006 -5.499989) (xy 3.080004 -5.499989) (xy 3.080004 -3.499993) (xy 3.580003 -3.499993) (xy 2.580005 -2.499995)
    (xy 1.580007 -3.499993) (xy 2.080006 -3.499993) (xy 2.080006 -5.499989))
   (stroke (width 0) (type solid)) (fill yes) (layer "F.SilkS"))
  (pad "1" thru_hole circle (at -2.54 0 90) (size 2 2) (drill 1.300022) (layers "*.Cu" "*.Mask") (remove_unused_layers no) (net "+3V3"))
  (pad "2" thru_hole circle (at 2.54 0 90) (size 2 2) (drill 1.300022) (layers "*.Cu" "*.Mask") (remove_unused_layers no) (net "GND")))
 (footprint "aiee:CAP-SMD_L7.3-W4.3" (layer "F.Cu") (at 23.5515 25.9525 -90)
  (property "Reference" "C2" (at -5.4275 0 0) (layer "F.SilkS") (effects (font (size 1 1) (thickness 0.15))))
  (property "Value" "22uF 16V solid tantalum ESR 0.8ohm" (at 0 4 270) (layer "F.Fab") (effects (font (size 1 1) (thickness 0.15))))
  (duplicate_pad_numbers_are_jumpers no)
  (fp_line (start -3.81 2.29) (end 3.81 2.29) (stroke (width 0.15) (type solid)) (layer "F.SilkS"))
  (fp_line (start 3.81 2.29) (end 3.81 2.03) (stroke (width 0.15) (type solid)) (layer "F.SilkS"))
  (fp_line (start -3.81 2.03) (end -3.81 2.29) (stroke (width 0.15) (type solid)) (layer "F.SilkS"))
  (fp_line (start 3.81 -2.03) (end 3.81 -2.29) (stroke (width 0.15) (type solid)) (layer "F.SilkS"))
  (fp_line (start 2.2 -2.23) (end 2.2 2.23) (stroke (width 0.15) (type solid)) (layer "F.SilkS"))
  (fp_line (start -3.81 -2.29) (end -3.81 -2.16) (stroke (width 0.15) (type solid)) (layer "F.SilkS"))
  (fp_line (start 3.81 -2.29) (end -3.81 -2.29) (stroke (width 0.15) (type solid)) (layer "F.SilkS"))
  (fp_circle (center 3.65 -2.15) (end 3.68 -2.15) (stroke (width 0.15) (type solid)) (fill no) (layer "F.SilkS"))
  (pad "1" smd rect (at 3.41 0 90) (size 2.185 3.78) (layers "F.Cu" "F.Mask" "F.Paste") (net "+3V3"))
  (pad "2" smd rect (at -3.41 0 90) (size 2.185 3.78) (layers "F.Cu" "F.Mask" "F.Paste") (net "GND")))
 (gr_rect (start 5.125 19.7) (end 39.78 54.355) (stroke (width 0.1) (type default)) (fill no) (layer "Edge.Cuts"))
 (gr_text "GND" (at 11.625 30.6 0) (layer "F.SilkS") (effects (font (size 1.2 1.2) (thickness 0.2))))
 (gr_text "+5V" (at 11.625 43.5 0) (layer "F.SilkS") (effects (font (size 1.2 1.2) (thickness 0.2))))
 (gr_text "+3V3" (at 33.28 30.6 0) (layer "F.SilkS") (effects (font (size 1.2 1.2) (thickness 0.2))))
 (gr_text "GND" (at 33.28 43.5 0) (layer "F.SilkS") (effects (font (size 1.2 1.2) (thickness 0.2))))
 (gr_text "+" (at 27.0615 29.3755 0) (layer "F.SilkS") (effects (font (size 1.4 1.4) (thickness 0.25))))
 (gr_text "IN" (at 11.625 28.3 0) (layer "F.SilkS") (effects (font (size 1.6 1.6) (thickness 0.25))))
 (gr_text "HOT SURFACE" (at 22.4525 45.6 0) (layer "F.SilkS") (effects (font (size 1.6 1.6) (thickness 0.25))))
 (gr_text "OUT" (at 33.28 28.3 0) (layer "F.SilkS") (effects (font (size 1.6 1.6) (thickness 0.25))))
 (segment (start 22.1 22.5425) (end 21.1115 22.5425) (width 0.6) (layer "F.Cu") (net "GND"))
 (segment (start 18.9 30.045) (end 17.9535 30.045) (width 0.6) (layer "F.Cu") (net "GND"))
 (segment (start 25 22.5425) (end 25.9915 22.5425) (width 0.6) (layer "F.Cu") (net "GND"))
 (segment (start 26 32.605) (end 26.9515 32.605) (width 0.6) (layer "F.Cu") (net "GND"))
 (segment (start 26.1 31.7) (end 26.1 30.805) (width 0.6) (layer "F.Cu") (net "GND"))
 (via (at 25.9915 22.5425) (size 0.6) (drill 0.3) (layers "F.Cu" "B.Cu") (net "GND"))
 (via (at 26.1 30.805) (size 0.6) (drill 0.3) (layers "F.Cu" "B.Cu") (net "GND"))
 (via (at 21.1115 22.5425) (size 0.6) (drill 0.3) (layers "F.Cu" "B.Cu") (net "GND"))
 (via (at 26.9515 32.605) (size 0.6) (drill 0.3) (layers "F.Cu" "B.Cu") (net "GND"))
 (via (at 17.9535 30.045) (size 0.6) (drill 0.3) (layers "F.Cu" "B.Cu") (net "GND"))
 (segment (start 19.65 32.6) (end 21.25 32.6) (width 0.3862) (layer "F.Cu") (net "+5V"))
 (segment (start 19.15 33.1) (end 12.7 39.55) (width 0.3862) (layer "F.Cu") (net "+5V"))
 (segment (start 12.7 39.55) (end 11.6 39.55) (width 0.3862) (layer "F.Cu") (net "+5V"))
 (segment (start 19.15 33.1) (end 19.65 32.6) (width 0.3862) (layer "F.Cu") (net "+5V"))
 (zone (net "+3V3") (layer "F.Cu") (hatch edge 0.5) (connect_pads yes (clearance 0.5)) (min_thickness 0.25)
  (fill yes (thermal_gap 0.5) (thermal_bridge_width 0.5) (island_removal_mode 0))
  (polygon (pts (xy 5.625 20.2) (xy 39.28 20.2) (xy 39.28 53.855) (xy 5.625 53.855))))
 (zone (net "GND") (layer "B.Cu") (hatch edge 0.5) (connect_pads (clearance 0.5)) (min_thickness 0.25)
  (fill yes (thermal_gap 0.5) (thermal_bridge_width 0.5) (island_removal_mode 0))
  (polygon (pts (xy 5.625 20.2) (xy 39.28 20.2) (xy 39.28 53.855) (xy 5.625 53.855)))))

